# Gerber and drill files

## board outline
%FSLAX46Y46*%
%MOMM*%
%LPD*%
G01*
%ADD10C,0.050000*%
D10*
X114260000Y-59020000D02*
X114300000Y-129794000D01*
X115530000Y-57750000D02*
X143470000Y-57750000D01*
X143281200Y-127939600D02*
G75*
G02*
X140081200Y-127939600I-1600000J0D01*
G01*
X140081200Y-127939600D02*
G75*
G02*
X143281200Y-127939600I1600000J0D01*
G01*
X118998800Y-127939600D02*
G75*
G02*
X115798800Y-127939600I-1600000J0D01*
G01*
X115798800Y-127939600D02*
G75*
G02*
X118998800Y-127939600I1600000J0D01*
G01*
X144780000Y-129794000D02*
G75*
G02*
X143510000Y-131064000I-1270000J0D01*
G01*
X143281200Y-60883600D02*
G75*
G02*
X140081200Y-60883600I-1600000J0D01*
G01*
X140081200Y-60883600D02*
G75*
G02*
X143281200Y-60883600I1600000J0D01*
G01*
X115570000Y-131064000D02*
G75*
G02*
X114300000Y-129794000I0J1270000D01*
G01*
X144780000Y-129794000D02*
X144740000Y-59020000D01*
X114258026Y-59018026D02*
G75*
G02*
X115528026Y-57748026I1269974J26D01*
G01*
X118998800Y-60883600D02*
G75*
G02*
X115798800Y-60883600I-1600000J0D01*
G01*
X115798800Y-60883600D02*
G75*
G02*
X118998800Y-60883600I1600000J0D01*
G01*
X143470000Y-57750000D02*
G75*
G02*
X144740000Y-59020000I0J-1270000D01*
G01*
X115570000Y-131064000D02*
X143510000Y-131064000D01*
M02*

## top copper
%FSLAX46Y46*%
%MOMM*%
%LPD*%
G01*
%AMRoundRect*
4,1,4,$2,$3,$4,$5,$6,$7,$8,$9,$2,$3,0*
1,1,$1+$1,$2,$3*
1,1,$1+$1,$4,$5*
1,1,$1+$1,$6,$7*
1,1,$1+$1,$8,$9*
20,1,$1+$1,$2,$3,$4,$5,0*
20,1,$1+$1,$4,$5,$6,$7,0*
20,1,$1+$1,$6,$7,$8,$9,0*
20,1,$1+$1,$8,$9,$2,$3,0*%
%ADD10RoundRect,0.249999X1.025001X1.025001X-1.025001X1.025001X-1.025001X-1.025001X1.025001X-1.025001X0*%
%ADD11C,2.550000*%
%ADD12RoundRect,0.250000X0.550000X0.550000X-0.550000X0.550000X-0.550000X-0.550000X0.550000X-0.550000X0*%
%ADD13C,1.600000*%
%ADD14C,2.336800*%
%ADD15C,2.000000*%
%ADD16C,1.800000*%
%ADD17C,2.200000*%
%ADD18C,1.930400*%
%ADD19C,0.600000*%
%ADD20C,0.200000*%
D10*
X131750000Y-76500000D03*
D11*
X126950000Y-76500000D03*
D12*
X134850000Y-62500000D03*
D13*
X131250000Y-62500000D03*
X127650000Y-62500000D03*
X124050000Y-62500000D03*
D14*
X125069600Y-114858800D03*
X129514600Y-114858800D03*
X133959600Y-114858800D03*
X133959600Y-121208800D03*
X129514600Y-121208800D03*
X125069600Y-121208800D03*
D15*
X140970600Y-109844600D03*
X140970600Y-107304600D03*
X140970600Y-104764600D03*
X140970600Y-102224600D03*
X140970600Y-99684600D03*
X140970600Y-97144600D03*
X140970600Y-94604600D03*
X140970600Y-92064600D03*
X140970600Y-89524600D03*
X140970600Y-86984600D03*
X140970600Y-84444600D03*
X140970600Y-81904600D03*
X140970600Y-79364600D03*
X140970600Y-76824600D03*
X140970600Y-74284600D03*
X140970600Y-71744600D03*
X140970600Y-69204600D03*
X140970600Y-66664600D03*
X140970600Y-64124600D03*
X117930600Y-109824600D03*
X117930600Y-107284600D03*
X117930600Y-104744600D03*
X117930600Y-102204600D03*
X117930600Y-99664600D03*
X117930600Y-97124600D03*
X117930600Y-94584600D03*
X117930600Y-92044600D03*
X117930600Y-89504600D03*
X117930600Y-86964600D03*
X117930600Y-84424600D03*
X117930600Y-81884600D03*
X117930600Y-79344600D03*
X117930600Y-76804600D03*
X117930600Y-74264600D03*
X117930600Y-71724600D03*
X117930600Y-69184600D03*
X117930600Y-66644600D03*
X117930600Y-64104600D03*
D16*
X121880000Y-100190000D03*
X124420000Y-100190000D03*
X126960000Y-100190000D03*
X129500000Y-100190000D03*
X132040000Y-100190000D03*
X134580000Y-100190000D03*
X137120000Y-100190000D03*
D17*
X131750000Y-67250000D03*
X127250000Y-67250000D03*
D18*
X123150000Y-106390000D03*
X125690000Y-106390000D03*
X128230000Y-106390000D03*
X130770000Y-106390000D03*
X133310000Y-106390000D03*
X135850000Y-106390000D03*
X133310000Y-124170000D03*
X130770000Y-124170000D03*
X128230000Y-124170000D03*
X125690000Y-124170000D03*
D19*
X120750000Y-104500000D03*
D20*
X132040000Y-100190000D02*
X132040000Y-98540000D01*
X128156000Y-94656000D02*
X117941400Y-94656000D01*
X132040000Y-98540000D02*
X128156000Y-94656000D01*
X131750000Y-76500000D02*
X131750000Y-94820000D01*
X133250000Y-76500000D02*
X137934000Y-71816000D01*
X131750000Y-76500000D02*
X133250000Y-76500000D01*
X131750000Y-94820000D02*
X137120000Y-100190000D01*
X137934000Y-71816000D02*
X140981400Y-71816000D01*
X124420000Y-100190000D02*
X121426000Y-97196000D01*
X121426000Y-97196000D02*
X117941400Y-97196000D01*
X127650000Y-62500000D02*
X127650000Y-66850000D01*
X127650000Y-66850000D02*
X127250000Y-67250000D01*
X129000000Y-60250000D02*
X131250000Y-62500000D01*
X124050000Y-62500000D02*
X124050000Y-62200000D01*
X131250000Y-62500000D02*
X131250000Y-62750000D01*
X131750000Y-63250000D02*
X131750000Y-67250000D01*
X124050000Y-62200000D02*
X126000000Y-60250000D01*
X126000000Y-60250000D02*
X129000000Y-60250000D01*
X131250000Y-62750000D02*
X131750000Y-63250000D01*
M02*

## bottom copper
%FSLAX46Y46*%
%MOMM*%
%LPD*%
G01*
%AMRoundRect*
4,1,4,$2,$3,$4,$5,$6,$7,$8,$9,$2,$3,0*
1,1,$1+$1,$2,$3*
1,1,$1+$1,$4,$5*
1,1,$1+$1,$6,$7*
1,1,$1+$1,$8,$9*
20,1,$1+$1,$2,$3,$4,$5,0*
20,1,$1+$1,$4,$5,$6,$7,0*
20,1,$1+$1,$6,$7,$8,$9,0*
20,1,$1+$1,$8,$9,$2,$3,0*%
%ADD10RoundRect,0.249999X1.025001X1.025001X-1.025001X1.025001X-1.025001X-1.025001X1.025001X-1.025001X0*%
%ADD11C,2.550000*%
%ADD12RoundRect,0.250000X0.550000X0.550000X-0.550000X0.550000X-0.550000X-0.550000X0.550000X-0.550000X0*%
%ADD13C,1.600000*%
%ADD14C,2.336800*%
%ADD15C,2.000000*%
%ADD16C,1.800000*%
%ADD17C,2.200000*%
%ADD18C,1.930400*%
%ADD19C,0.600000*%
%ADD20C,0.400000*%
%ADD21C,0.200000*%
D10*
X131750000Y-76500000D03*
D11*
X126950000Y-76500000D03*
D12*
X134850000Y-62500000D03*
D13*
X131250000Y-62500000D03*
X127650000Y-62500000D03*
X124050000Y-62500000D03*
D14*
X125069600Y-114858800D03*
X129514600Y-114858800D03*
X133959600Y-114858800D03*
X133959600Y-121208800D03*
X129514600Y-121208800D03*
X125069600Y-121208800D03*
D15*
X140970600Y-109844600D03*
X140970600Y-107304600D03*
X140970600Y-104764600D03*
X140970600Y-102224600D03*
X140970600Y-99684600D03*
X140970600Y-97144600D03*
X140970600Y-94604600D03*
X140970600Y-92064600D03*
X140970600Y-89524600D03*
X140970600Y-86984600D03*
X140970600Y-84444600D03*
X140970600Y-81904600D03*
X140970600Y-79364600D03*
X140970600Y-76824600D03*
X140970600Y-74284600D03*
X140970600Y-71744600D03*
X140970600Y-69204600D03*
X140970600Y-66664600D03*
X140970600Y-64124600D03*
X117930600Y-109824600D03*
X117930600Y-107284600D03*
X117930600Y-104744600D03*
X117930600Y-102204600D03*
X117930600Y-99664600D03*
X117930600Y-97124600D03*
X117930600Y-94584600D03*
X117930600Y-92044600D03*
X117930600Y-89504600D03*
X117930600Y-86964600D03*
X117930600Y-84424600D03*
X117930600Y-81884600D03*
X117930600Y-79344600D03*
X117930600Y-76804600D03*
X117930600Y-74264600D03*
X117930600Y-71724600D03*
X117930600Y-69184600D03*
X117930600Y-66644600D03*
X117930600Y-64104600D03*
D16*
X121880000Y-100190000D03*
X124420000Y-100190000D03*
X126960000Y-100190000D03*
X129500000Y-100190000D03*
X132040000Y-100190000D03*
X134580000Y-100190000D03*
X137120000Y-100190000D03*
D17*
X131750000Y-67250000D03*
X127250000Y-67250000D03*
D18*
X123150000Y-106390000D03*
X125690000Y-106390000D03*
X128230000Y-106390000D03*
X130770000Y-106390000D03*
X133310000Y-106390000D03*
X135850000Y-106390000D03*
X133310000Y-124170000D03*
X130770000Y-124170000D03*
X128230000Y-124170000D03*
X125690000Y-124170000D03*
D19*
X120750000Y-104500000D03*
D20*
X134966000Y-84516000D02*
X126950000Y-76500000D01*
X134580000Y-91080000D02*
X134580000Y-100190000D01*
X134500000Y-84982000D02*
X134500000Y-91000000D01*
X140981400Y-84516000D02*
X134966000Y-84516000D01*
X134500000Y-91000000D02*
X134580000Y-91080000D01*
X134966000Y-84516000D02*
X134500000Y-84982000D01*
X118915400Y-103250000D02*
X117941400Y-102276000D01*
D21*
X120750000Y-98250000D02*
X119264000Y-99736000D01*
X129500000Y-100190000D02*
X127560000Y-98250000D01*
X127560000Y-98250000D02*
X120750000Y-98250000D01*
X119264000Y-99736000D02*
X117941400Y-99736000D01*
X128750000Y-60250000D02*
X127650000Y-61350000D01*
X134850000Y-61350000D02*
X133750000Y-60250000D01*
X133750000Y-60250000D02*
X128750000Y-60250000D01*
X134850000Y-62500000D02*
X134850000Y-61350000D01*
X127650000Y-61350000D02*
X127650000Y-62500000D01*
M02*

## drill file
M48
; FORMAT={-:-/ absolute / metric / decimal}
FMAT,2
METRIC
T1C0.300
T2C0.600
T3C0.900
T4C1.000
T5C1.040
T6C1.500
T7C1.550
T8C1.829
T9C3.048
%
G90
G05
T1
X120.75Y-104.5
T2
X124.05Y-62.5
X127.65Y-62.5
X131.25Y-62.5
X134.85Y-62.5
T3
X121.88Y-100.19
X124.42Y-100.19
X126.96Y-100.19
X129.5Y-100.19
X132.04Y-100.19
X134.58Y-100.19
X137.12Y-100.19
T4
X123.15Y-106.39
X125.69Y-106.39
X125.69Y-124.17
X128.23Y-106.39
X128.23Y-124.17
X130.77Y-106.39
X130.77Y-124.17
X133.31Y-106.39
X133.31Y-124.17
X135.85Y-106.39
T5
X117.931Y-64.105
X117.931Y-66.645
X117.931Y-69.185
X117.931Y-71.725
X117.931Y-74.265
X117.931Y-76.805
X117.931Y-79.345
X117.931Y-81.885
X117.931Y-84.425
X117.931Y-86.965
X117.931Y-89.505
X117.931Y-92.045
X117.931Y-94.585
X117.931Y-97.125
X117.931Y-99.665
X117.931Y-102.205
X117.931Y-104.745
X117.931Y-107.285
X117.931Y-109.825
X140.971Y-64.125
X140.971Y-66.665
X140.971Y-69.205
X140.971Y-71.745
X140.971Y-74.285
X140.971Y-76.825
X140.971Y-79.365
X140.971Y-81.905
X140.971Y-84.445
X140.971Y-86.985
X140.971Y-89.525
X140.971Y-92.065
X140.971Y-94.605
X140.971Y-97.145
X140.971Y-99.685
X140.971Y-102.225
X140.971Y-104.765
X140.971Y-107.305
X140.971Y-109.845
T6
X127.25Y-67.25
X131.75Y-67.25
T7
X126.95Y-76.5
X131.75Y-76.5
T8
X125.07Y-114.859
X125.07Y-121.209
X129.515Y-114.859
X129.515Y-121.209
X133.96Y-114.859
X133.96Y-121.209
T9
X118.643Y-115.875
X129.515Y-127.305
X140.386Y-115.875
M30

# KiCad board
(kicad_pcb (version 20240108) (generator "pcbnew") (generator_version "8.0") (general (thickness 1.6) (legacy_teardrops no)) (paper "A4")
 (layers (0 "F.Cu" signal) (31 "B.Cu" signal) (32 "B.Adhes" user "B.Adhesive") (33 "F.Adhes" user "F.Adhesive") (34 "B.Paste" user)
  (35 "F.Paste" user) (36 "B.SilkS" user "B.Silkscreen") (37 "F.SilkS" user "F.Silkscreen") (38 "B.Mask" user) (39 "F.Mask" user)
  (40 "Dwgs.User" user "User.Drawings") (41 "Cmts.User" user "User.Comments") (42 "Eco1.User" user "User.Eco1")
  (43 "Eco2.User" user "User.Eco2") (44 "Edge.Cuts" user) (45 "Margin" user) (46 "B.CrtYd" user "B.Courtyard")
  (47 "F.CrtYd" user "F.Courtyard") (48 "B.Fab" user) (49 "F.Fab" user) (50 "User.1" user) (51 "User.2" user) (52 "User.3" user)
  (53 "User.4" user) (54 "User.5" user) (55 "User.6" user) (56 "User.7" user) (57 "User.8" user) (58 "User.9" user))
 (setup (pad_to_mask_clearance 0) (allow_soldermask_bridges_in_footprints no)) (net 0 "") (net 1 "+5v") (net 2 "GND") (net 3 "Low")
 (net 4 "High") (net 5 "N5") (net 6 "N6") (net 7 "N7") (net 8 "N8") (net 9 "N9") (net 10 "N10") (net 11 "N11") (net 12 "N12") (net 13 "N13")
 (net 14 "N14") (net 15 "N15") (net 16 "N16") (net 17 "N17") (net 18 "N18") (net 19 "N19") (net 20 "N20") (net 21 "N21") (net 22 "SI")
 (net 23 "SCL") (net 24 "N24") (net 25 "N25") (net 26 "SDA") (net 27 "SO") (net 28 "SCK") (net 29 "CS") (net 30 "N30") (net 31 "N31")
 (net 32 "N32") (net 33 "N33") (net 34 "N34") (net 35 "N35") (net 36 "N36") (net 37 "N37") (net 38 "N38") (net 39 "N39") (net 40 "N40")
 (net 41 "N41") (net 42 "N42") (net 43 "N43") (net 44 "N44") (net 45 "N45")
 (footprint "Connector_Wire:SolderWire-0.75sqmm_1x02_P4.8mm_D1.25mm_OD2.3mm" (layer "F.Cu") (at 131.75 76.5 180)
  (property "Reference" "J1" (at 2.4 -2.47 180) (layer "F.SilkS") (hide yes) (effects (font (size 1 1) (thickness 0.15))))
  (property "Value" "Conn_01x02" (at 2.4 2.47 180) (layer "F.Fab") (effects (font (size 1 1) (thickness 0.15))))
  (pad "1" thru_hole roundrect (at 0 0 180) (size 2.55 2.55) (drill 1.55) (layers "*.Cu" "*.Mask") (remove_unused_layers no)
   (roundrect_rratio 0.098039) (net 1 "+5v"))
  (pad "2" thru_hole circle (at 4.8 0 180) (size 2.55 2.55) (drill 1.55) (layers "*.Cu" "*.Mask") (remove_unused_layers no) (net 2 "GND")))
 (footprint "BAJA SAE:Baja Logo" (layer "F.Cu") (at 129 114)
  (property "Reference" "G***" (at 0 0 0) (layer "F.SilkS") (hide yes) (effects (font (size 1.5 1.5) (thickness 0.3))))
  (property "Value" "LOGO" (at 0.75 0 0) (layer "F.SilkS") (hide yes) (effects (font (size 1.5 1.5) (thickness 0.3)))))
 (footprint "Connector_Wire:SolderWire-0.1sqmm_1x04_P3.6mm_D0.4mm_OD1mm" (layer "F.Cu") (at 134.85 62.5 180)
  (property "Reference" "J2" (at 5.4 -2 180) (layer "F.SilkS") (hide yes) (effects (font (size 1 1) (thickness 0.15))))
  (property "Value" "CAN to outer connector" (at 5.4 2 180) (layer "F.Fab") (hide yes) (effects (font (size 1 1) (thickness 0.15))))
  (pad "1" thru_hole roundrect (at 0 0 180) (size 1.6 1.6) (drill 0.6) (layers "*.Cu" "*.Mask") (remove_unused_layers no)
   (roundrect_rratio 0.15625) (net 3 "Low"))
  (pad "2" thru_hole circle (at 3.6 0 180) (size 1.6 1.6) (drill 0.6) (layers "*.Cu" "*.Mask") (remove_unused_layers no) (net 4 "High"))
  (pad "3" thru_hole circle (at 7.2 0 180) (size 1.6 1.6) (drill 0.6) (layers "*.Cu" "*.Mask") (remove_unused_layers no) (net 3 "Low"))
  (pad "4" thru_hole circle (at 10.8 0 180) (size 1.6 1.6) (drill 0.6) (layers "*.Cu" "*.Mask") (remove_unused_layers no) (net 4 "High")))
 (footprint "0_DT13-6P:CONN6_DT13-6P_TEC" (layer "F.Cu") (at 125.0696 114.8588 180)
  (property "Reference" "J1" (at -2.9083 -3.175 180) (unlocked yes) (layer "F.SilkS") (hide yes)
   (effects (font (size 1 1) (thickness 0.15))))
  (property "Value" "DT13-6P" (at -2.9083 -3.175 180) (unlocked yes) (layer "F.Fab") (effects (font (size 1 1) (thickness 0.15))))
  (pad "" np_thru_hole circle (at -15.3162 -1.016 180) (size 3.048 3.048) (drill 3.048) (layers))
  (pad "" np_thru_hole circle (at -4.445 -12.446 180) (size 3.048 3.048) (drill 3.048) (layers))
  (pad "" np_thru_hole circle (at 6.4262 -1.016 180) (size 3.048 3.048) (drill 3.048) (layers))
  (pad "1" thru_hole circle (at 0 0 180) (size 2.3368 2.3368) (drill 1.8288) (layers "*.Cu" "*.Mask") (remove_unused_layers no)
   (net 1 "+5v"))
  (pad "2" thru_hole circle (at -4.445 0 180) (size 2.3368 2.3368) (drill 1.8288) (layers "*.Cu" "*.Mask") (remove_unused_layers no)
   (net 2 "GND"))
  (pad "3" thru_hole circle (at -8.89 0 180) (size 2.3368 2.3368) (drill 1.8288) (layers "*.Cu" "*.Mask") (remove_unused_layers no)
   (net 3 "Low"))
  (pad "4" thru_hole circle (at -8.89 -6.35 180) (size 2.3368 2.3368) (drill 1.8288) (layers "*.Cu" "*.Mask") (remove_unused_layers no)
   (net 4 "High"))
  (pad "5" thru_hole circle (at -4.445 -6.35 180) (size 2.3368 2.3368) (drill 1.8288) (layers "*.Cu" "*.Mask") (remove_unused_layers no)
   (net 3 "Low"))
  (pad "6" thru_hole circle (at 0 -6.35 180) (size 2.3368 2.3368) (drill 1.8288) (layers "*.Cu" "*.Mask") (remove_unused_layers no)
   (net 4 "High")))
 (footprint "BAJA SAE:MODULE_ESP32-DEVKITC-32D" (layer "F.Cu") (at 129.2106 90.9146 180)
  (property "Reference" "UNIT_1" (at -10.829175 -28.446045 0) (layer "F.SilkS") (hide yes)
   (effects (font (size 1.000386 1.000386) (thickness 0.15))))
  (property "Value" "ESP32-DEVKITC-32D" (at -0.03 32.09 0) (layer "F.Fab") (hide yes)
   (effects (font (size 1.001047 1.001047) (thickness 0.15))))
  (pad "J2-1" thru_hole circle (at -11.76 -18.93 180) (size 2 2) (drill 1.04) (layers "*.Cu" "*.Mask") (remove_unused_layers no)
   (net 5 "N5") (solder_mask_margin 0.102))
  (pad "J2-2" thru_hole circle (at -11.76 -16.39 180) (size 2 2) (drill 1.04) (layers "*.Cu" "*.Mask") (remove_unused_layers no)
   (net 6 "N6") (solder_mask_margin 0.102))
  (pad "J2-3" thru_hole circle (at -11.76 -13.85 180) (size 2 2) (drill 1.04) (layers "*.Cu" "*.Mask") (remove_unused_layers no)
   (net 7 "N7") (solder_mask_margin 0.102))
  (pad "J2-4" thru_hole circle (at -11.76 -11.31 180) (size 2 2) (drill 1.04) (layers "*.Cu" "*.Mask") (remove_unused_layers no)
   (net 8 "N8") (solder_mask_margin 0.102))
  (pad "J2-5" thru_hole circle (at -11.76 -8.77 180) (size 2 2) (drill 1.04) (layers "*.Cu" "*.Mask") (remove_unused_layers no) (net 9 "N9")
   (solder_mask_margin 0.102))
  (pad "J2-6" thru_hole circle (at -11.76 -6.23 180) (size 2 2) (drill 1.04) (layers "*.Cu" "*.Mask") (remove_unused_layers no)
   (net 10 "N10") (solder_mask_margin 0.102))
  (pad "J2-7" thru_hole circle (at -11.76 -3.69 180) (size 2 2) (drill 1.04) (layers "*.Cu" "*.Mask") (remove_unused_layers no)
   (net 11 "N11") (solder_mask_margin 0.102))
  (pad "J2-8" thru_hole circle (at -11.76 -1.15 180) (size 2 2) (drill 1.04) (layers "*.Cu" "*.Mask") (remove_unused_layers no)
   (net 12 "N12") (solder_mask_margin 0.102))
  (pad "J2-9" thru_hole circle (at -11.76 1.39 180) (size 2 2) (drill 1.04) (layers "*.Cu" "*.Mask") (remove_unused_layers no)
   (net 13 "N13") (solder_mask_margin 0.102))
  (pad "J2-10" thru_hole circle (at -11.76 3.93 180) (size 2 2) (drill 1.04) (layers "*.Cu" "*.Mask") (remove_unused_layers no)
   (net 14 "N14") (solder_mask_margin 0.102))
  (pad "J2-11" thru_hole circle (at -11.76 6.47 180) (size 2 2) (drill 1.04) (layers "*.Cu" "*.Mask") (remove_unused_layers no)
   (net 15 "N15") (solder_mask_margin 0.102))
  (pad "J2-12" thru_hole circle (at -11.76 9.01 180) (size 2 2) (drill 1.04) (layers "*.Cu" "*.Mask") (remove_unused_layers no)
   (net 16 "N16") (solder_mask_margin 0.102))
  (pad "J2-13" thru_hole circle (at -11.76 11.55 180) (size 2 2) (drill 1.04) (layers "*.Cu" "*.Mask") (remove_unused_layers no)
   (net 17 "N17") (solder_mask_margin 0.102))
  (pad "J2-14" thru_hole circle (at -11.76 14.09 180) (size 2 2) (drill 1.04) (layers "*.Cu" "*.Mask") (remove_unused_layers no)
   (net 2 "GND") (solder_mask_margin 0.102))
  (pad "J2-15" thru_hole circle (at -11.76 16.63 180) (size 2 2) (drill 1.04) (layers "*.Cu" "*.Mask") (remove_unused_layers no)
   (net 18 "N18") (solder_mask_margin 0.102))
  (pad "J2-16" thru_hole circle (at -11.76 19.17 180) (size 2 2) (drill 1.04) (layers "*.Cu" "*.Mask") (remove_unused_layers no)
   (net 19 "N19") (solder_mask_margin 0.102))
  (pad "J2-17" thru_hole circle (at -11.76 21.71 180) (size 2 2) (drill 1.04) (layers "*.Cu" "*.Mask") (remove_unused_layers no)
   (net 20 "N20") (solder_mask_margin 0.102))
  (pad "J2-18" thru_hole circle (at -11.76 24.25 180) (size 2 2) (drill 1.04) (layers "*.Cu" "*.Mask") (remove_unused_layers no)
   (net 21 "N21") (solder_mask_margin 0.102))
  (pad "J2-19" thru_hole circle (at -11.76 26.79 180) (size 2 2) (drill 1.04) (layers "*.Cu" "*.Mask") (remove_unused_layers no)
   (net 1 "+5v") (solder_mask_margin 0.102))
  (pad "J3-1" thru_hole circle (at 11.28 -18.91 180) (size 2 2) (drill 1.04) (layers "*.Cu" "*.Mask") (remove_unused_layers no)
   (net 2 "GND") (solder_mask_margin 0.102))
  (pad "J3-2" thru_hole circle (at 11.28 -16.37 180) (size 2 2) (drill 1.04) (layers "*.Cu" "*.Mask") (remove_unused_layers no)
   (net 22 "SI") (solder_mask_margin 0.102))
  (pad "J3-3" thru_hole circle (at 11.28 -13.83 180) (size 2 2) (drill 1.04) (layers "*.Cu" "*.Mask") (remove_unused_layers no)
   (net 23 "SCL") (solder_mask_margin 0.102))
  (pad "J3-4" thru_hole circle (at 11.28 -11.29 180) (size 2 2) (drill 1.04) (layers "*.Cu" "*.Mask") (remove_unused_layers no)
   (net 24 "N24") (solder_mask_margin 0.102))
  (pad "J3-5" thru_hole circle (at 11.28 -8.75 180) (size 2 2) (drill 1.04) (layers "*.Cu" "*.Mask") (remove_unused_layers no)
   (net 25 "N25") (solder_mask_margin 0.102))
  (pad "J3-6" thru_hole circle (at 11.28 -6.21 180) (size 2 2) (drill 1.04) (layers "*.Cu" "*.Mask") (remove_unused_layers no)
   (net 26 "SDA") (solder_mask_margin 0.102))
  (pad "J3-7" thru_hole circle (at 11.28 -3.67 180) (size 2 2) (drill 1.04) (layers "*.Cu" "*.Mask") (remove_unused_layers no) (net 2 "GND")
   (solder_mask_margin 0.102))
  (pad "J3-8" thru_hole circle (at 11.28 -1.13 180) (size 2 2) (drill 1.04) (layers "*.Cu" "*.Mask") (remove_unused_layers no) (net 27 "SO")
   (solder_mask_margin 0.102))
  (pad "J3-9" thru_hole circle (at 11.28 1.41 180) (size 2 2) (drill 1.04) (layers "*.Cu" "*.Mask") (remove_unused_layers no) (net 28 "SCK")
   (solder_mask_margin 0.102))
  (pad "J3-10" thru_hole circle (at 11.28 3.95 180) (size 2 2) (drill 1.04) (layers "*.Cu" "*.Mask") (remove_unused_layers no) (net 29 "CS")
   (solder_mask_margin 0.102))
  (pad "J3-11" thru_hole circle (at 11.28 6.49 180) (size 2 2) (drill 1.04) (layers "*.Cu" "*.Mask") (remove_unused_layers no)
   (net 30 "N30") (solder_mask_margin 0.102))
  (pad "J3-12" thru_hole circle (at 11.28 9.03 180) (size 2 2) (drill 1.04) (layers "*.Cu" "*.Mask") (remove_unused_layers no)
   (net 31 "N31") (solder_mask_margin 0.102))
  (pad "J3-13" thru_hole circle (at 11.28 11.57 180) (size 2 2) (drill 1.04) (layers "*.Cu" "*.Mask") (remove_unused_layers no)
   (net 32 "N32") (solder_mask_margin 0.102))
  (pad "J3-14" thru_hole circle (at 11.28 14.11 180) (size 2 2) (drill 1.04) (layers "*.Cu" "*.Mask") (remove_unused_layers no)
   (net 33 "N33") (solder_mask_margin 0.102))
  (pad "J3-15" thru_hole circle (at 11.28 16.65 180) (size 2 2) (drill 1.04) (layers "*.Cu" "*.Mask") (remove_unused_layers no)
   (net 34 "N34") (solder_mask_margin 0.102))
  (pad "J3-16" thru_hole circle (at 11.28 19.19 180) (size 2 2) (drill 1.04) (layers "*.Cu" "*.Mask") (remove_unused_layers no)
   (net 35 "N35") (solder_mask_margin 0.102))
  (pad "J3-17" thru_hole circle (at 11.28 21.73 180) (size 2 2) (drill 1.04) (layers "*.Cu" "*.Mask") (remove_unused_layers no)
   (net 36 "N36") (solder_mask_margin 0.102))
  (pad "J3-18" thru_hole circle (at 11.28 24.27 180) (size 2 2) (drill 1.04) (layers "*.Cu" "*.Mask") (remove_unused_layers no)
   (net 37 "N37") (solder_mask_margin 0.102))
  (pad "J3-19" thru_hole circle (at 11.28 26.81 180) (size 2 2) (drill 1.04) (layers "*.Cu" "*.Mask") (remove_unused_layers no)
   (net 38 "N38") (solder_mask_margin 0.102)))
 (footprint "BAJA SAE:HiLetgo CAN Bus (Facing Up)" (layer "B.Cu") (at 127.1 90.24 90)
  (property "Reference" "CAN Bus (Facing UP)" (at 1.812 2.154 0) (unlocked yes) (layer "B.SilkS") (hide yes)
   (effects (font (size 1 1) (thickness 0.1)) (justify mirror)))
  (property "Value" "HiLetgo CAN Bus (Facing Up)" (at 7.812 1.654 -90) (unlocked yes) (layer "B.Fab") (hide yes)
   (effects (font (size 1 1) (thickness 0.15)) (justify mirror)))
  (pad "1" thru_hole circle (at -9.95 -5.22 270) (size 1.8 1.8) (drill 0.9) (layers "*.Cu" "*.Mask") (remove_unused_layers no)
   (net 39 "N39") (solder_mask_margin 0.102))
  (pad "2" thru_hole circle (at -9.95 -2.68 270) (size 1.8 1.8) (drill 0.9) (layers "*.Cu" "*.Mask") (remove_unused_layers no)
   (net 28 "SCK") (solder_mask_margin 0.102))
  (pad "3" thru_hole circle (at -9.95 -0.14 270) (size 1.8 1.8) (drill 0.9) (layers "*.Cu" "*.Mask") (remove_unused_layers no) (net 22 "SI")
   (solder_mask_margin 0.102))
  (pad "4" thru_hole circle (at -9.95 2.4 270) (size 1.8 1.8) (drill 0.9) (layers "*.Cu" "*.Mask") (remove_unused_layers no) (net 27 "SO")
   (solder_mask_margin 0.102))
  (pad "5" thru_hole circle (at -9.95 4.94 270) (size 1.8 1.8) (drill 0.9) (layers "*.Cu" "*.Mask") (remove_unused_layers no) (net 29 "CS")
   (solder_mask_margin 0.102))
  (pad "6" thru_hole circle (at -9.95 7.48 270) (size 1.8 1.8) (drill 0.9) (layers "*.Cu" "*.Mask") (remove_unused_layers no) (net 2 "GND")
   (solder_mask_margin 0.102))
  (pad "7" thru_hole circle (at -9.95 10.02 270) (size 1.8 1.8) (drill 0.9) (layers "*.Cu" "*.Mask") (remove_unused_layers no) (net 1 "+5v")
   (solder_mask_margin 0.102))
  (pad "8" thru_hole circle (at 22.99 4.65 270) (size 2.2 2.2) (drill 1.5) (layers "*.Cu" "*.Mask") (remove_unused_layers no) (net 4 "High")
   (solder_mask_margin 0.102))
  (pad "9" thru_hole circle (at 22.99 0.15 270) (size 2.2 2.2) (drill 1.5) (layers "*.Cu" "*.Mask") (remove_unused_layers no) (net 3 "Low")
   (solder_mask_margin 0.102)))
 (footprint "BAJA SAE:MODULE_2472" (layer "B.Cu") (at 129.5 115.28)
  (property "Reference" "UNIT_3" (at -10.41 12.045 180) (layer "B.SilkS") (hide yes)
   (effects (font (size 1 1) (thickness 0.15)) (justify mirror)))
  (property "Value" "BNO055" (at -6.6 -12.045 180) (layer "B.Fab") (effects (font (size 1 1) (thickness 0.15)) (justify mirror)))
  (pad "1" thru_hole circle (at -6.35 -8.89) (size 1.9304 1.9304) (drill 1) (layers "*.Cu" "*.Mask") (remove_unused_layers no) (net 1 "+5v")
   (solder_mask_margin 0.102))
  (pad "2" thru_hole circle (at -3.81 -8.89) (size 1.9304 1.9304) (drill 1) (layers "*.Cu" "*.Mask") (remove_unused_layers no)
   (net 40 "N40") (solder_mask_margin 0.102))
  (pad "3" thru_hole circle (at -1.27 -8.89) (size 1.9304 1.9304) (drill 1) (layers "*.Cu" "*.Mask") (remove_unused_layers no) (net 2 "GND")
   (solder_mask_margin 0.102))
  (pad "4" thru_hole circle (at 1.27 -8.89) (size 1.9304 1.9304) (drill 1) (layers "*.Cu" "*.Mask") (remove_unused_layers no) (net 26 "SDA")
   (solder_mask_margin 0.102))
  (pad "5" thru_hole circle (at 3.81 -8.89) (size 1.9304 1.9304) (drill 1) (layers "*.Cu" "*.Mask") (remove_unused_layers no) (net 23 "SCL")
   (solder_mask_margin 0.102))
  (pad "6" thru_hole circle (at 6.35 -8.89) (size 1.9304 1.9304) (drill 1) (layers "*.Cu" "*.Mask") (remove_unused_layers no) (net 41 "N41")
   (solder_mask_margin 0.102))
  (pad "7" thru_hole circle (at 3.81 8.89) (size 1.9304 1.9304) (drill 1) (layers "*.Cu" "*.Mask") (remove_unused_layers no) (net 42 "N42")
   (solder_mask_margin 0.102))
  (pad "8" thru_hole circle (at 1.27 8.89) (size 1.9304 1.9304) (drill 1) (layers "*.Cu" "*.Mask") (remove_unused_layers no) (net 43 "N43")
   (solder_mask_margin 0.102))
  (pad "9" thru_hole circle (at -1.27 8.89) (size 1.9304 1.9304) (drill 1) (layers "*.Cu" "*.Mask") (remove_unused_layers no) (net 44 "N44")
   (solder_mask_margin 0.102))
  (pad "10" thru_hole circle (at -3.81 8.89) (size 1.9304 1.9304) (drill 1) (layers "*.Cu" "*.Mask") (remove_unused_layers no)
   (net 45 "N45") (solder_mask_margin 0.102)))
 (gr_line (start 114.26 59.02) (end 114.3 129.794) (locked yes) (stroke (width 0.05) (type default)) (layer "Edge.Cuts"))
 (gr_line (start 115.53 57.75) (end 143.47 57.75) (locked yes) (stroke (width 0.05) (type default)) (layer "Edge.Cuts"))
 (gr_circle (center 141.6812 127.9396) (end 143.2812 127.9396) (stroke (width 0.05) (type default)) (fill none) (layer "Edge.Cuts"))
 (gr_circle (center 117.3988 127.9396) (end 118.9988 127.9396) (stroke (width 0.05) (type default)) (fill none) (layer "Edge.Cuts"))
 (gr_arc (start 144.78 129.794) (mid 144.408026 130.692026) (end 143.51 131.064) (stroke (width 0.05) (type default)) (layer "Edge.Cuts"))
 (gr_circle (center 141.6812 60.8836) (end 143.2812 60.8836) (stroke (width 0.05) (type default)) (fill none) (layer "Edge.Cuts"))
 (gr_arc (start 115.57 131.064) (mid 114.671974 130.692026) (end 114.3 129.794) (stroke (width 0.05) (type default)) (layer "Edge.Cuts"))
 (gr_line (start 144.78 129.794) (end 144.74 59.02) (stroke (width 0.05) (type default)) (layer "Edge.Cuts"))
 (gr_arc (start 114.258026 59.018026) (mid 114.63 58.12) (end 115.528026 57.748026) (stroke (width 0.05) (type default)) (layer "Edge.Cuts"))
 (gr_circle (center 117.3988 60.8836) (end 118.9988 60.8836) (stroke (width 0.05) (type default)) (fill none) (layer "Edge.Cuts"))
 (gr_arc (start 143.47 57.75) (mid 144.368026 58.121974) (end 144.74 59.02) (stroke (width 0.05) (type default)) (layer "Edge.Cuts"))
 (gr_line (start 115.57 131.064) (end 143.51 131.064) (stroke (width 0.05) (type default)) (layer "Edge.Cuts"))
 (segment (start 134.966 84.516) (end 126.95 76.5) (width 0.4) (layer "B.Cu") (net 2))
 (segment (start 134.58 91.08) (end 134.58 100.19) (width 0.4) (layer "B.Cu") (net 2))
 (segment (start 134.5 84.982) (end 134.5 91) (width 0.4) (layer "B.Cu") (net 2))
 (segment (start 140.9814 84.516) (end 134.966 84.516) (width 0.4) (layer "B.Cu") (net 2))
 (segment (start 134.5 91) (end 134.58 91.08) (width 0.4) (layer "B.Cu") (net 2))
 (segment (start 134.966 84.516) (end 134.5 84.982) (width 0.4) (layer "B.Cu") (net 2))
 (segment (start 118.9154 103.25) (end 117.9414 102.276) (width 0.4) (layer "B.Cu") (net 24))
 (via (at 120.75 104.5) (size 0.6) (drill 0.3) (layers "F.Cu" "B.Cu") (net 22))
 (segment (start 132.04 100.19) (end 132.04 98.54) (width 0.2) (layer "F.Cu") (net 29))
 (segment (start 128.156 94.656) (end 117.9414 94.656) (width 0.2) (layer "F.Cu") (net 29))
 (segment (start 132.04 98.54) (end 128.156 94.656) (width 0.2) (layer "F.Cu") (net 29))
 (segment (start 131.75 76.5) (end 131.75 94.82) (width 0.2) (layer "F.Cu") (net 1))
 (segment (start 133.25 76.5) (end 137.934 71.816) (width 0.2) (layer "F.Cu") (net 1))
 (segment (start 131.75 76.5) (end 133.25 76.5) (width 0.2) (layer "F.Cu") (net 1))
 (segment (start 131.75 94.82) (end 137.12 100.19) (width 0.2) (layer "F.Cu") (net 1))
 (segment (start 137.934 71.816) (end 140.9814 71.816) (width 0.2) (layer "F.Cu") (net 1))
 (segment (start 124.42 100.19) (end 121.426 97.196) (width 0.2) (layer "F.Cu") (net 28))
 (segment (start 121.426 97.196) (end 117.9414 97.196) (width 0.2) (layer "F.Cu") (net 28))
 (segment (start 120.75 98.25) (end 119.264 99.736) (width 0.2) (layer "B.Cu") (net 27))
 (segment (start 129.5 100.19) (end 127.56 98.25) (width 0.2) (layer "B.Cu") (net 27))
 (segment (start 127.56 98.25) (end 120.75 98.25) (width 0.2) (layer "B.Cu") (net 27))
 (segment (start 119.264 99.736) (end 117.9414 99.736) (width 0.2) (layer "B.Cu") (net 27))
 (segment (start 127.65 62.5) (end 127.65 66.85) (width 0.2) (layer "F.Cu") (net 3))
 (segment (start 127.65 66.85) (end 127.25 67.25) (width 0.2) (layer "F.Cu") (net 3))
 (segment (start 128.75 60.25) (end 127.65 61.35) (width 0.2) (layer "B.Cu") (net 3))
 (segment (start 134.85 61.35) (end 133.75 60.25) (width 0.2) (layer "B.Cu") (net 3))
 (segment (start 133.75 60.25) (end 128.75 60.25) (width 0.2) (layer "B.Cu") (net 3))
 (segment (start 134.85 62.5) (end 134.85 61.35) (width 0.2) (layer "B.Cu") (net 3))
 (segment (start 127.65 61.35) (end 127.65 62.5) (width 0.2) (layer "B.Cu") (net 3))
 (segment (start 129 60.25) (end 131.25 62.5) (width 0.2) (layer "F.Cu") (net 4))
 (segment (start 124.05 62.5) (end 124.05 62.2) (width 0.2) (layer "F.Cu") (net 4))
 (segment (start 131.25 62.5) (end 131.25 62.75) (width 0.2) (layer "F.Cu") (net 4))
 (segment (start 131.75 63.25) (end 131.75 67.25) (width 0.2) (layer "F.Cu") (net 4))
 (segment (start 124.05 62.2) (end 126 60.25) (width 0.2) (layer "F.Cu") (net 4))
 (segment (start 126 60.25) (end 129 60.25) (width 0.2) (layer "F.Cu") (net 4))
 (segment (start 131.25 62.75) (end 131.75 63.25) (width 0.2) (layer "F.Cu") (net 4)))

